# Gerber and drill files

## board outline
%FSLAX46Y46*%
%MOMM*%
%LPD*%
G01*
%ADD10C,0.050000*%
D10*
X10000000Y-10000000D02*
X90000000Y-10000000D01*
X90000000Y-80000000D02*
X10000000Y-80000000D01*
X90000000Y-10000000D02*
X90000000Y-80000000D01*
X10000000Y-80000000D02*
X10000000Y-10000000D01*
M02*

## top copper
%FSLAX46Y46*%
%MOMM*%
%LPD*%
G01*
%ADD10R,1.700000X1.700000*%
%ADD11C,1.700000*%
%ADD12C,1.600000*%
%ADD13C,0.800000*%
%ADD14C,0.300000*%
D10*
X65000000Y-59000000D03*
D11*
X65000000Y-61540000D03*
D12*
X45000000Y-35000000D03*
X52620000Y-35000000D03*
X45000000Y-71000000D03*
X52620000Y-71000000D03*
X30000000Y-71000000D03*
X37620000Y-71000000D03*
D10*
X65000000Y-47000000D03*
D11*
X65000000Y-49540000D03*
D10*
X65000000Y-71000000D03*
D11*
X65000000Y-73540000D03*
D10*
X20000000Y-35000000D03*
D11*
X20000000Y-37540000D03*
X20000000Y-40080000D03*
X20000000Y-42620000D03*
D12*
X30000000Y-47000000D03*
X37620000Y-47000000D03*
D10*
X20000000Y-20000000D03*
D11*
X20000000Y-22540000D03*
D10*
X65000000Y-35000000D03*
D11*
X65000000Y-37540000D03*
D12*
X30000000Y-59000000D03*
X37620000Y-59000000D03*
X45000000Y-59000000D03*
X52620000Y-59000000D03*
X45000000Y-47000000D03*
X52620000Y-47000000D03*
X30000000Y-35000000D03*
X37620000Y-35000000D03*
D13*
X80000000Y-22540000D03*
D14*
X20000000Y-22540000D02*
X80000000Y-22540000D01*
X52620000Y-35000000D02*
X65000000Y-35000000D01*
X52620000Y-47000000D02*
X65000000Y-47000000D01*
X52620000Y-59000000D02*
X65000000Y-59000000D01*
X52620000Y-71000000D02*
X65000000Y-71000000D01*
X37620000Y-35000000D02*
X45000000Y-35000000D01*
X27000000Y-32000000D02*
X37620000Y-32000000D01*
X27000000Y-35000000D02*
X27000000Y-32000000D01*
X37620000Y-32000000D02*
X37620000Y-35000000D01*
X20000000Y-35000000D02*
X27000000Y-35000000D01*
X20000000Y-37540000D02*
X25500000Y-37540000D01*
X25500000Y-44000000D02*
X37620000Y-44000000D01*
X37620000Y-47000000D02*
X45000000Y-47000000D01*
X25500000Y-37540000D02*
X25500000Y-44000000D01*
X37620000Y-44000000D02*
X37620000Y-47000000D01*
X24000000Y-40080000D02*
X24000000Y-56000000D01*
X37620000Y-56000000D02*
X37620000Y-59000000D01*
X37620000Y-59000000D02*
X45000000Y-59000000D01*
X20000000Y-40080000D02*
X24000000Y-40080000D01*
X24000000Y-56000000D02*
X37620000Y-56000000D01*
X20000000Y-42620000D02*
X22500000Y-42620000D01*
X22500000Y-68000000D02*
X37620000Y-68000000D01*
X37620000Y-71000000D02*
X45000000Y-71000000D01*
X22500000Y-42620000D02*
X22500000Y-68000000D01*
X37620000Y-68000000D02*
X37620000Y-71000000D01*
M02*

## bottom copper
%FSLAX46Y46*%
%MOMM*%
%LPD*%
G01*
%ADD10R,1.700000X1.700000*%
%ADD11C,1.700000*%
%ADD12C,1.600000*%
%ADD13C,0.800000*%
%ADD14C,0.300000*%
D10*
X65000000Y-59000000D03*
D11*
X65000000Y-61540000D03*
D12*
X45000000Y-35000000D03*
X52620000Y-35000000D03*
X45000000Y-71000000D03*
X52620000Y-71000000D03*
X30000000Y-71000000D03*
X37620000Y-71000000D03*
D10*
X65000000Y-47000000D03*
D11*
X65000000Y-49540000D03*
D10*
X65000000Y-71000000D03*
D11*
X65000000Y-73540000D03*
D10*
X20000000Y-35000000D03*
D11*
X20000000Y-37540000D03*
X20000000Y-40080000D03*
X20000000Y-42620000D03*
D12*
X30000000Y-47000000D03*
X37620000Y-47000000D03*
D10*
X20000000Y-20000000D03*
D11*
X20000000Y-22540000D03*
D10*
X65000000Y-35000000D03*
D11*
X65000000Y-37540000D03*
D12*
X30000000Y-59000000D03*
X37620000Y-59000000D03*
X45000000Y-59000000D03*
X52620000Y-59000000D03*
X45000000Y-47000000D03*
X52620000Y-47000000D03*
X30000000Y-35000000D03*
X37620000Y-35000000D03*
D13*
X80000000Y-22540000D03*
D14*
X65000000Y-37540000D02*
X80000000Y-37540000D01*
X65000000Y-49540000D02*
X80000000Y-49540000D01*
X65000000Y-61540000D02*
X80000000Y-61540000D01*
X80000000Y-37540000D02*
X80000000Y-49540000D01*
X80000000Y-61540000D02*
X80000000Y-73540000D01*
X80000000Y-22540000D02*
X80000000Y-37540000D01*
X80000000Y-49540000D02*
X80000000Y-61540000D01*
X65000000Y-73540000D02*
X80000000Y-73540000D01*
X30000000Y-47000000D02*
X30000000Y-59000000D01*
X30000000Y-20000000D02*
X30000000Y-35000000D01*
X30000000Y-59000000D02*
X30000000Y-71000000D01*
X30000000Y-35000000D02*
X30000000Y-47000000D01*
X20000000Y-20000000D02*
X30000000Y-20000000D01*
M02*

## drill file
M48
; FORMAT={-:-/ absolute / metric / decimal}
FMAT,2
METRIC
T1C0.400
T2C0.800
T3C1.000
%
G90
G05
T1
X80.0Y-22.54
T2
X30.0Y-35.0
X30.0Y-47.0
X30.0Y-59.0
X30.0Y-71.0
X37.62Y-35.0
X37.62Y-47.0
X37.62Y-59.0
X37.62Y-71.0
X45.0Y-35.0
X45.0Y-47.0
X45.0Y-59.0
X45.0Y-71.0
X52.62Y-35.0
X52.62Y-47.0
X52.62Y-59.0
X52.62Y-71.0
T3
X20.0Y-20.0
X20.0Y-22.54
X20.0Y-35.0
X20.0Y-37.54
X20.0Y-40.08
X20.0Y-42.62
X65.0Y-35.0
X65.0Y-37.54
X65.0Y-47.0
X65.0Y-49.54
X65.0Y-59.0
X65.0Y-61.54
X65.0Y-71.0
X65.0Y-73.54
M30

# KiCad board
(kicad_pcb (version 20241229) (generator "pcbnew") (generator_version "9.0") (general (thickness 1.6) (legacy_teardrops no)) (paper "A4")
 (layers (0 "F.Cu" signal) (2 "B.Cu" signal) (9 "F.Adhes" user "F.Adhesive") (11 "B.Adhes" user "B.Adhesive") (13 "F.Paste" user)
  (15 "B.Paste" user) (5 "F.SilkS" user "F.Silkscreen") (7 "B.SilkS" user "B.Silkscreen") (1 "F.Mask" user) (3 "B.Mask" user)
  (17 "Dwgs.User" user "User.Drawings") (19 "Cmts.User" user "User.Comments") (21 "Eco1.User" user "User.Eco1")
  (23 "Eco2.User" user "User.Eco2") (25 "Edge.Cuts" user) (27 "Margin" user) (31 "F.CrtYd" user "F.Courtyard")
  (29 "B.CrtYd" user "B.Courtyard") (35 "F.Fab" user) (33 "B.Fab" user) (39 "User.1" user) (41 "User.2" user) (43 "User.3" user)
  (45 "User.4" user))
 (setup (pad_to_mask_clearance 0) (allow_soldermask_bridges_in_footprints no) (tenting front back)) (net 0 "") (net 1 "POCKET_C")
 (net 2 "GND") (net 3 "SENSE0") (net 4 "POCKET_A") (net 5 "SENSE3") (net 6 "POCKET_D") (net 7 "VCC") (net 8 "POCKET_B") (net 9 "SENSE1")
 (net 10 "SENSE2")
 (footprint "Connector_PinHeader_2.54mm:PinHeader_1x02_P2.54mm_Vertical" (layer "F.Cu") (at 65 59)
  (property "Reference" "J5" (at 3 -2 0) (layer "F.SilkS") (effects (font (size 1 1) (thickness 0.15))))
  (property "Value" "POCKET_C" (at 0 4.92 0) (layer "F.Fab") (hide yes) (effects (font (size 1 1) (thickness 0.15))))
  (pad "1" thru_hole rect (at 0 0) (size 1.7 1.7) (drill 1) (layers "*.Cu" "*.Mask") (remove_unused_layers no) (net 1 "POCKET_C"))
  (pad "2" thru_hole circle (at 0 2.54) (size 1.7 1.7) (drill 1) (layers "*.Cu" "*.Mask") (remove_unused_layers no) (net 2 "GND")))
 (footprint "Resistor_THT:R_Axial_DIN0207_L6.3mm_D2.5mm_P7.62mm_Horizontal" (layer "F.Cu") (at 45 35)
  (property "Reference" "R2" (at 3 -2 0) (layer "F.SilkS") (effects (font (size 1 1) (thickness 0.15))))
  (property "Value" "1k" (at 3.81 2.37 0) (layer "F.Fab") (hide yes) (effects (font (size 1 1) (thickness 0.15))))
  (pad "1" thru_hole circle (at 0 0) (size 1.6 1.6) (drill 0.8) (layers "*.Cu" "*.Mask") (remove_unused_layers no) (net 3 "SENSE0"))
  (pad "2" thru_hole circle (at 7.62 0) (size 1.6 1.6) (drill 0.8) (layers "*.Cu" "*.Mask") (remove_unused_layers no) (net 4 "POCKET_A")))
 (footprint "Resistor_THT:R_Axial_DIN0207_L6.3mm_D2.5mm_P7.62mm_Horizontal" (layer "F.Cu") (at 45 71)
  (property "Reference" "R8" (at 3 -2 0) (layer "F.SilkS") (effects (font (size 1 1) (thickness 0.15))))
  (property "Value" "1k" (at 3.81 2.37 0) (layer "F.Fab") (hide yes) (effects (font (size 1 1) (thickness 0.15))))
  (pad "1" thru_hole circle (at 0 0) (size 1.6 1.6) (drill 0.8) (layers "*.Cu" "*.Mask") (remove_unused_layers no) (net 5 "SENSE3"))
  (pad "2" thru_hole circle (at 7.62 0) (size 1.6 1.6) (drill 0.8) (layers "*.Cu" "*.Mask") (remove_unused_layers no) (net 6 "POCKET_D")))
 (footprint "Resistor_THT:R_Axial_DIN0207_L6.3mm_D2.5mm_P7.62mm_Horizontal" (layer "F.Cu") (at 30 71)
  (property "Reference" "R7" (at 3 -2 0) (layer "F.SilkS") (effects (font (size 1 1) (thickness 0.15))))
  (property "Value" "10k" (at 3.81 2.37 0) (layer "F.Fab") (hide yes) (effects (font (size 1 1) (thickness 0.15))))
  (pad "1" thru_hole circle (at 0 0) (size 1.6 1.6) (drill 0.8) (layers "*.Cu" "*.Mask") (remove_unused_layers no) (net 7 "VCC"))
  (pad "2" thru_hole circle (at 7.62 0) (size 1.6 1.6) (drill 0.8) (layers "*.Cu" "*.Mask") (remove_unused_layers no) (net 5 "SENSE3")))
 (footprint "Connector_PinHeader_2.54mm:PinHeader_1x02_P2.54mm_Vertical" (layer "F.Cu") (at 65 47)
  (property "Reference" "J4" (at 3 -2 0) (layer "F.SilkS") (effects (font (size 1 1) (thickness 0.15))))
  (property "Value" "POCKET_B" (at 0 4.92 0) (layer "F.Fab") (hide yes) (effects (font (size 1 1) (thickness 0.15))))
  (pad "1" thru_hole rect (at 0 0) (size 1.7 1.7) (drill 1) (layers "*.Cu" "*.Mask") (remove_unused_layers no) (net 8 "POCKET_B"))
  (pad "2" thru_hole circle (at 0 2.54) (size 1.7 1.7) (drill 1) (layers "*.Cu" "*.Mask") (remove_unused_layers no) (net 2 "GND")))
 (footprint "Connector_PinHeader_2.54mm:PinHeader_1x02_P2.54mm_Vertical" (layer "F.Cu") (at 65 71)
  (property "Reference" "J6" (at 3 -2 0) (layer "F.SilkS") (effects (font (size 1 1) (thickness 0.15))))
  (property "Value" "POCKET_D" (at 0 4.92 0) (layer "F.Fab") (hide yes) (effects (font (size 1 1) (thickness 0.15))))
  (pad "1" thru_hole rect (at 0 0) (size 1.7 1.7) (drill 1) (layers "*.Cu" "*.Mask") (remove_unused_layers no) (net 6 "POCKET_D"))
  (pad "2" thru_hole circle (at 0 2.54) (size 1.7 1.7) (drill 1) (layers "*.Cu" "*.Mask") (remove_unused_layers no) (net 2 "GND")))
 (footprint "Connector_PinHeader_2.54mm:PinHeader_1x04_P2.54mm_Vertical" (layer "F.Cu") (at 20 35)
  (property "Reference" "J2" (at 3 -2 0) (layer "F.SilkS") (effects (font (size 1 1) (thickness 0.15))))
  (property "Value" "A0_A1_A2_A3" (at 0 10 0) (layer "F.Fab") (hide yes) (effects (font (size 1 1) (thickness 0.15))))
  (pad "1" thru_hole rect (at 0 0) (size 1.7 1.7) (drill 1) (layers "*.Cu" "*.Mask") (remove_unused_layers no) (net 3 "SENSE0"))
  (pad "2" thru_hole circle (at 0 2.54) (size 1.7 1.7) (drill 1) (layers "*.Cu" "*.Mask") (remove_unused_layers no) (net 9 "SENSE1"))
  (pad "3" thru_hole circle (at 0 5.08) (size 1.7 1.7) (drill 1) (layers "*.Cu" "*.Mask") (remove_unused_layers no) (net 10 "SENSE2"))
  (pad "4" thru_hole circle (at 0 7.62) (size 1.7 1.7) (drill 1) (layers "*.Cu" "*.Mask") (remove_unused_layers no) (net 5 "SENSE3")))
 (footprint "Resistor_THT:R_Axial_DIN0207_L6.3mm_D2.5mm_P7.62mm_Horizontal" (layer "F.Cu") (at 30 47)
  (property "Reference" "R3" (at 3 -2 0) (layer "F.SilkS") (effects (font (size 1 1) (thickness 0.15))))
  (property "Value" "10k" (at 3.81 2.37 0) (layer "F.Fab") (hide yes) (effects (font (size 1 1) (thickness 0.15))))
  (pad "1" thru_hole circle (at 0 0) (size 1.6 1.6) (drill 0.8) (layers "*.Cu" "*.Mask") (remove_unused_layers no) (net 7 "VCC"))
  (pad "2" thru_hole circle (at 7.62 0) (size 1.6 1.6) (drill 0.8) (layers "*.Cu" "*.Mask") (remove_unused_layers no) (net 9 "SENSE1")))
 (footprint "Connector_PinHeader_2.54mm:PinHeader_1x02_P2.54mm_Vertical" (layer "F.Cu") (at 20 20)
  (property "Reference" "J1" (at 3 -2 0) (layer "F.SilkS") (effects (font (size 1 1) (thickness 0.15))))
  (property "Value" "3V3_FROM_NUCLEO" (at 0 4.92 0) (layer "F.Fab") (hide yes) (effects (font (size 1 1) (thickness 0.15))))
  (pad "1" thru_hole rect (at 0 0) (size 1.7 1.7) (drill 1) (layers "*.Cu" "*.Mask") (remove_unused_layers no) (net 7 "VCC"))
  (pad "2" thru_hole circle (at 0 2.54) (size 1.7 1.7) (drill 1) (layers "*.Cu" "*.Mask") (remove_unused_layers no) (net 2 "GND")))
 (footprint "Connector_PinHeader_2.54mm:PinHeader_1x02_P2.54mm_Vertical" (layer "F.Cu") (at 65 35)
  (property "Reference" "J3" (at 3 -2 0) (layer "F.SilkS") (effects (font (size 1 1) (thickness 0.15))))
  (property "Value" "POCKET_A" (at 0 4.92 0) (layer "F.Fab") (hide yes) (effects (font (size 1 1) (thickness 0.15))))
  (pad "1" thru_hole rect (at 0 0) (size 1.7 1.7) (drill 1) (layers "*.Cu" "*.Mask") (remove_unused_layers no) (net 4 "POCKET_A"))
  (pad "2" thru_hole circle (at 0 2.54) (size 1.7 1.7) (drill 1) (layers "*.Cu" "*.Mask") (remove_unused_layers no) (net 2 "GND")))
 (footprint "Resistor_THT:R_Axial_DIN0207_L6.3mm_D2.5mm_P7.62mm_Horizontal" (layer "F.Cu") (at 30 59)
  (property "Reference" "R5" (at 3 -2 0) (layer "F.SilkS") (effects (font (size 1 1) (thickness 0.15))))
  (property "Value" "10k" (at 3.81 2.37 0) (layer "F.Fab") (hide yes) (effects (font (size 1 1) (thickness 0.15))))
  (pad "1" thru_hole circle (at 0 0) (size 1.6 1.6) (drill 0.8) (layers "*.Cu" "*.Mask") (remove_unused_layers no) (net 7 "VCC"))
  (pad "2" thru_hole circle (at 7.62 0) (size 1.6 1.6) (drill 0.8) (layers "*.Cu" "*.Mask") (remove_unused_layers no) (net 10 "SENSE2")))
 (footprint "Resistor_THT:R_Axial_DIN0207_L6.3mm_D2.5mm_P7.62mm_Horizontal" (layer "F.Cu") (at 45 59)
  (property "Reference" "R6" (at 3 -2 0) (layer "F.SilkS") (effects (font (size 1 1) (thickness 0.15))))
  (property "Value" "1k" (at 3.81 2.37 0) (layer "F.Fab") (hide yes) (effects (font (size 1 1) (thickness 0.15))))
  (pad "1" thru_hole circle (at 0 0) (size 1.6 1.6) (drill 0.8) (layers "*.Cu" "*.Mask") (remove_unused_layers no) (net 10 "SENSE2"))
  (pad "2" thru_hole circle (at 7.62 0) (size 1.6 1.6) (drill 0.8) (layers "*.Cu" "*.Mask") (remove_unused_layers no) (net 1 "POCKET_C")))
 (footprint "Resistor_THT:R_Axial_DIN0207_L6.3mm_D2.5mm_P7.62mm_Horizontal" (layer "F.Cu") (at 45 47)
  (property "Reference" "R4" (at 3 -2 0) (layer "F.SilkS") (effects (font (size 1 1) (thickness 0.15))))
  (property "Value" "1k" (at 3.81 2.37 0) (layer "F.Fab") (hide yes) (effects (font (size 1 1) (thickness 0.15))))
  (pad "1" thru_hole circle (at 0 0) (size 1.6 1.6) (drill 0.8) (layers "*.Cu" "*.Mask") (remove_unused_layers no) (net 9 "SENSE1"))
  (pad "2" thru_hole circle (at 7.62 0) (size 1.6 1.6) (drill 0.8) (layers "*.Cu" "*.Mask") (remove_unused_layers no) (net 8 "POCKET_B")))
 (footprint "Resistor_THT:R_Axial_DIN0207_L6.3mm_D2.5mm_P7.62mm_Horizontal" (layer "F.Cu") (at 30 35)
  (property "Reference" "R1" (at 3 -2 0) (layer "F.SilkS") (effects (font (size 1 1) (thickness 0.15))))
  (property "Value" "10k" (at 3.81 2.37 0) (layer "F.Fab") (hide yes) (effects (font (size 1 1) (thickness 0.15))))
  (pad "1" thru_hole circle (at 0 0) (size 1.6 1.6) (drill 0.8) (layers "*.Cu" "*.Mask") (remove_unused_layers no) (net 7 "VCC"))
  (pad "2" thru_hole circle (at 7.62 0) (size 1.6 1.6) (drill 0.8) (layers "*.Cu" "*.Mask") (remove_unused_layers no) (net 3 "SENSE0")))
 (gr_line (start 10 10) (end 90 10) (stroke (width 0.05) (type default)) (layer "Edge.Cuts"))
 (gr_line (start 90 80) (end 10 80) (stroke (width 0.05) (type default)) (layer "Edge.Cuts"))
 (gr_line (start 90 10) (end 90 80) (stroke (width 0.05) (type default)) (layer "Edge.Cuts"))
 (gr_line (start 10 80) (end 10 10) (stroke (width 0.05) (type default)) (layer "Edge.Cuts"))
 (segment (start 20 22.54) (end 80 22.54) (width 0.3) (layer "F.Cu") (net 2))
 (via (at 80 22.54) (size 0.8) (drill 0.4) (layers "F.Cu" "B.Cu") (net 2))
 (segment (start 65 37.54) (end 80 37.54) (width 0.3) (layer "B.Cu") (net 2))
 (segment (start 65 49.54) (end 80 49.54) (width 0.3) (layer "B.Cu") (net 2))
 (segment (start 65 61.54) (end 80 61.54) (width 0.3) (layer "B.Cu") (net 2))
 (segment (start 80 37.54) (end 80 49.54) (width 0.3) (layer "B.Cu") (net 2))
 (segment (start 80 61.54) (end 80 73.54) (width 0.3) (layer "B.Cu") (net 2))
 (segment (start 80 22.54) (end 80 37.54) (width 0.3) (layer "B.Cu") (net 2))
 (segment (start 80 49.54) (end 80 61.54) (width 0.3) (layer "B.Cu") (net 2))
 (segment (start 65 73.54) (end 80 73.54) (width 0.3) (layer "B.Cu") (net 2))
 (segment (start 52.62 35) (end 65 35) (width 0.3) (layer "F.Cu") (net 4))
 (segment (start 52.62 47) (end 65 47) (width 0.3) (layer "F.Cu") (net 8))
 (segment (start 52.62 59) (end 65 59) (width 0.3) (layer "F.Cu") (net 1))
 (segment (start 52.62 71) (end 65 71) (width 0.3) (layer "F.Cu") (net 6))
 (segment (start 37.62 35) (end 45 35) (width 0.3) (layer "F.Cu") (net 3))
 (segment (start 27 32) (end 37.62 32) (width 0.3) (layer "F.Cu") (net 3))
 (segment (start 27 35) (end 27 32) (width 0.3) (layer "F.Cu") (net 3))
 (segment (start 37.62 32) (end 37.62 35) (width 0.3) (layer "F.Cu") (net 3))
 (segment (start 20 35) (end 27 35) (width 0.3) (layer "F.Cu") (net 3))
 (segment (start 20 37.54) (end 25.5 37.54) (width 0.3) (layer "F.Cu") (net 9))
 (segment (start 25.5 44) (end 37.62 44) (width 0.3) (layer "F.Cu") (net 9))
 (segment (start 37.62 47) (end 45 47) (width 0.3) (layer "F.Cu") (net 9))
 (segment (start 25.5 37.54) (end 25.5 44) (width 0.3) (layer "F.Cu") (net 9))
 (segment (start 37.62 44) (end 37.62 47) (width 0.3) (layer "F.Cu") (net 9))
 (segment (start 24 40.08) (end 24 56) (width 0.3) (layer "F.Cu") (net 10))
 (segment (start 37.62 56) (end 37.62 59) (width 0.3) (layer "F.Cu") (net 10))
 (segment (start 37.62 59) (end 45 59) (width 0.3) (layer "F.Cu") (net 10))
 (segment (start 20 40.08) (end 24 40.08) (width 0.3) (layer "F.Cu") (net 10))
 (segment (start 24 56) (end 37.62 56) (width 0.3) (layer "F.Cu") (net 10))
 (segment (start 20 42.62) (end 22.5 42.62) (width 0.3) (layer "F.Cu") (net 5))
 (segment (start 22.5 68) (end 37.62 68) (width 0.3) (layer "F.Cu") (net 5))
 (segment (start 37.62 71) (end 45 71) (width 0.3) (layer "F.Cu") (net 5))
 (segment (start 22.5 42.62) (end 22.5 68) (width 0.3) (layer "F.Cu") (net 5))
 (segment (start 37.62 68) (end 37.62 71) (width 0.3) (layer "F.Cu") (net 5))
 (segment (start 30 47) (end 30 59) (width 0.3) (layer "B.Cu") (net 7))
 (segment (start 30 20) (end 30 35) (width 0.3) (layer "B.Cu") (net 7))
 (segment (start 30 59) (end 30 71) (width 0.3) (layer "B.Cu") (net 7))
 (segment (start 30 35) (end 30 47) (width 0.3) (layer "B.Cu") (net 7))
 (segment (start 20 20) (end 30 20) (width 0.3) (layer "B.Cu") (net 7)))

